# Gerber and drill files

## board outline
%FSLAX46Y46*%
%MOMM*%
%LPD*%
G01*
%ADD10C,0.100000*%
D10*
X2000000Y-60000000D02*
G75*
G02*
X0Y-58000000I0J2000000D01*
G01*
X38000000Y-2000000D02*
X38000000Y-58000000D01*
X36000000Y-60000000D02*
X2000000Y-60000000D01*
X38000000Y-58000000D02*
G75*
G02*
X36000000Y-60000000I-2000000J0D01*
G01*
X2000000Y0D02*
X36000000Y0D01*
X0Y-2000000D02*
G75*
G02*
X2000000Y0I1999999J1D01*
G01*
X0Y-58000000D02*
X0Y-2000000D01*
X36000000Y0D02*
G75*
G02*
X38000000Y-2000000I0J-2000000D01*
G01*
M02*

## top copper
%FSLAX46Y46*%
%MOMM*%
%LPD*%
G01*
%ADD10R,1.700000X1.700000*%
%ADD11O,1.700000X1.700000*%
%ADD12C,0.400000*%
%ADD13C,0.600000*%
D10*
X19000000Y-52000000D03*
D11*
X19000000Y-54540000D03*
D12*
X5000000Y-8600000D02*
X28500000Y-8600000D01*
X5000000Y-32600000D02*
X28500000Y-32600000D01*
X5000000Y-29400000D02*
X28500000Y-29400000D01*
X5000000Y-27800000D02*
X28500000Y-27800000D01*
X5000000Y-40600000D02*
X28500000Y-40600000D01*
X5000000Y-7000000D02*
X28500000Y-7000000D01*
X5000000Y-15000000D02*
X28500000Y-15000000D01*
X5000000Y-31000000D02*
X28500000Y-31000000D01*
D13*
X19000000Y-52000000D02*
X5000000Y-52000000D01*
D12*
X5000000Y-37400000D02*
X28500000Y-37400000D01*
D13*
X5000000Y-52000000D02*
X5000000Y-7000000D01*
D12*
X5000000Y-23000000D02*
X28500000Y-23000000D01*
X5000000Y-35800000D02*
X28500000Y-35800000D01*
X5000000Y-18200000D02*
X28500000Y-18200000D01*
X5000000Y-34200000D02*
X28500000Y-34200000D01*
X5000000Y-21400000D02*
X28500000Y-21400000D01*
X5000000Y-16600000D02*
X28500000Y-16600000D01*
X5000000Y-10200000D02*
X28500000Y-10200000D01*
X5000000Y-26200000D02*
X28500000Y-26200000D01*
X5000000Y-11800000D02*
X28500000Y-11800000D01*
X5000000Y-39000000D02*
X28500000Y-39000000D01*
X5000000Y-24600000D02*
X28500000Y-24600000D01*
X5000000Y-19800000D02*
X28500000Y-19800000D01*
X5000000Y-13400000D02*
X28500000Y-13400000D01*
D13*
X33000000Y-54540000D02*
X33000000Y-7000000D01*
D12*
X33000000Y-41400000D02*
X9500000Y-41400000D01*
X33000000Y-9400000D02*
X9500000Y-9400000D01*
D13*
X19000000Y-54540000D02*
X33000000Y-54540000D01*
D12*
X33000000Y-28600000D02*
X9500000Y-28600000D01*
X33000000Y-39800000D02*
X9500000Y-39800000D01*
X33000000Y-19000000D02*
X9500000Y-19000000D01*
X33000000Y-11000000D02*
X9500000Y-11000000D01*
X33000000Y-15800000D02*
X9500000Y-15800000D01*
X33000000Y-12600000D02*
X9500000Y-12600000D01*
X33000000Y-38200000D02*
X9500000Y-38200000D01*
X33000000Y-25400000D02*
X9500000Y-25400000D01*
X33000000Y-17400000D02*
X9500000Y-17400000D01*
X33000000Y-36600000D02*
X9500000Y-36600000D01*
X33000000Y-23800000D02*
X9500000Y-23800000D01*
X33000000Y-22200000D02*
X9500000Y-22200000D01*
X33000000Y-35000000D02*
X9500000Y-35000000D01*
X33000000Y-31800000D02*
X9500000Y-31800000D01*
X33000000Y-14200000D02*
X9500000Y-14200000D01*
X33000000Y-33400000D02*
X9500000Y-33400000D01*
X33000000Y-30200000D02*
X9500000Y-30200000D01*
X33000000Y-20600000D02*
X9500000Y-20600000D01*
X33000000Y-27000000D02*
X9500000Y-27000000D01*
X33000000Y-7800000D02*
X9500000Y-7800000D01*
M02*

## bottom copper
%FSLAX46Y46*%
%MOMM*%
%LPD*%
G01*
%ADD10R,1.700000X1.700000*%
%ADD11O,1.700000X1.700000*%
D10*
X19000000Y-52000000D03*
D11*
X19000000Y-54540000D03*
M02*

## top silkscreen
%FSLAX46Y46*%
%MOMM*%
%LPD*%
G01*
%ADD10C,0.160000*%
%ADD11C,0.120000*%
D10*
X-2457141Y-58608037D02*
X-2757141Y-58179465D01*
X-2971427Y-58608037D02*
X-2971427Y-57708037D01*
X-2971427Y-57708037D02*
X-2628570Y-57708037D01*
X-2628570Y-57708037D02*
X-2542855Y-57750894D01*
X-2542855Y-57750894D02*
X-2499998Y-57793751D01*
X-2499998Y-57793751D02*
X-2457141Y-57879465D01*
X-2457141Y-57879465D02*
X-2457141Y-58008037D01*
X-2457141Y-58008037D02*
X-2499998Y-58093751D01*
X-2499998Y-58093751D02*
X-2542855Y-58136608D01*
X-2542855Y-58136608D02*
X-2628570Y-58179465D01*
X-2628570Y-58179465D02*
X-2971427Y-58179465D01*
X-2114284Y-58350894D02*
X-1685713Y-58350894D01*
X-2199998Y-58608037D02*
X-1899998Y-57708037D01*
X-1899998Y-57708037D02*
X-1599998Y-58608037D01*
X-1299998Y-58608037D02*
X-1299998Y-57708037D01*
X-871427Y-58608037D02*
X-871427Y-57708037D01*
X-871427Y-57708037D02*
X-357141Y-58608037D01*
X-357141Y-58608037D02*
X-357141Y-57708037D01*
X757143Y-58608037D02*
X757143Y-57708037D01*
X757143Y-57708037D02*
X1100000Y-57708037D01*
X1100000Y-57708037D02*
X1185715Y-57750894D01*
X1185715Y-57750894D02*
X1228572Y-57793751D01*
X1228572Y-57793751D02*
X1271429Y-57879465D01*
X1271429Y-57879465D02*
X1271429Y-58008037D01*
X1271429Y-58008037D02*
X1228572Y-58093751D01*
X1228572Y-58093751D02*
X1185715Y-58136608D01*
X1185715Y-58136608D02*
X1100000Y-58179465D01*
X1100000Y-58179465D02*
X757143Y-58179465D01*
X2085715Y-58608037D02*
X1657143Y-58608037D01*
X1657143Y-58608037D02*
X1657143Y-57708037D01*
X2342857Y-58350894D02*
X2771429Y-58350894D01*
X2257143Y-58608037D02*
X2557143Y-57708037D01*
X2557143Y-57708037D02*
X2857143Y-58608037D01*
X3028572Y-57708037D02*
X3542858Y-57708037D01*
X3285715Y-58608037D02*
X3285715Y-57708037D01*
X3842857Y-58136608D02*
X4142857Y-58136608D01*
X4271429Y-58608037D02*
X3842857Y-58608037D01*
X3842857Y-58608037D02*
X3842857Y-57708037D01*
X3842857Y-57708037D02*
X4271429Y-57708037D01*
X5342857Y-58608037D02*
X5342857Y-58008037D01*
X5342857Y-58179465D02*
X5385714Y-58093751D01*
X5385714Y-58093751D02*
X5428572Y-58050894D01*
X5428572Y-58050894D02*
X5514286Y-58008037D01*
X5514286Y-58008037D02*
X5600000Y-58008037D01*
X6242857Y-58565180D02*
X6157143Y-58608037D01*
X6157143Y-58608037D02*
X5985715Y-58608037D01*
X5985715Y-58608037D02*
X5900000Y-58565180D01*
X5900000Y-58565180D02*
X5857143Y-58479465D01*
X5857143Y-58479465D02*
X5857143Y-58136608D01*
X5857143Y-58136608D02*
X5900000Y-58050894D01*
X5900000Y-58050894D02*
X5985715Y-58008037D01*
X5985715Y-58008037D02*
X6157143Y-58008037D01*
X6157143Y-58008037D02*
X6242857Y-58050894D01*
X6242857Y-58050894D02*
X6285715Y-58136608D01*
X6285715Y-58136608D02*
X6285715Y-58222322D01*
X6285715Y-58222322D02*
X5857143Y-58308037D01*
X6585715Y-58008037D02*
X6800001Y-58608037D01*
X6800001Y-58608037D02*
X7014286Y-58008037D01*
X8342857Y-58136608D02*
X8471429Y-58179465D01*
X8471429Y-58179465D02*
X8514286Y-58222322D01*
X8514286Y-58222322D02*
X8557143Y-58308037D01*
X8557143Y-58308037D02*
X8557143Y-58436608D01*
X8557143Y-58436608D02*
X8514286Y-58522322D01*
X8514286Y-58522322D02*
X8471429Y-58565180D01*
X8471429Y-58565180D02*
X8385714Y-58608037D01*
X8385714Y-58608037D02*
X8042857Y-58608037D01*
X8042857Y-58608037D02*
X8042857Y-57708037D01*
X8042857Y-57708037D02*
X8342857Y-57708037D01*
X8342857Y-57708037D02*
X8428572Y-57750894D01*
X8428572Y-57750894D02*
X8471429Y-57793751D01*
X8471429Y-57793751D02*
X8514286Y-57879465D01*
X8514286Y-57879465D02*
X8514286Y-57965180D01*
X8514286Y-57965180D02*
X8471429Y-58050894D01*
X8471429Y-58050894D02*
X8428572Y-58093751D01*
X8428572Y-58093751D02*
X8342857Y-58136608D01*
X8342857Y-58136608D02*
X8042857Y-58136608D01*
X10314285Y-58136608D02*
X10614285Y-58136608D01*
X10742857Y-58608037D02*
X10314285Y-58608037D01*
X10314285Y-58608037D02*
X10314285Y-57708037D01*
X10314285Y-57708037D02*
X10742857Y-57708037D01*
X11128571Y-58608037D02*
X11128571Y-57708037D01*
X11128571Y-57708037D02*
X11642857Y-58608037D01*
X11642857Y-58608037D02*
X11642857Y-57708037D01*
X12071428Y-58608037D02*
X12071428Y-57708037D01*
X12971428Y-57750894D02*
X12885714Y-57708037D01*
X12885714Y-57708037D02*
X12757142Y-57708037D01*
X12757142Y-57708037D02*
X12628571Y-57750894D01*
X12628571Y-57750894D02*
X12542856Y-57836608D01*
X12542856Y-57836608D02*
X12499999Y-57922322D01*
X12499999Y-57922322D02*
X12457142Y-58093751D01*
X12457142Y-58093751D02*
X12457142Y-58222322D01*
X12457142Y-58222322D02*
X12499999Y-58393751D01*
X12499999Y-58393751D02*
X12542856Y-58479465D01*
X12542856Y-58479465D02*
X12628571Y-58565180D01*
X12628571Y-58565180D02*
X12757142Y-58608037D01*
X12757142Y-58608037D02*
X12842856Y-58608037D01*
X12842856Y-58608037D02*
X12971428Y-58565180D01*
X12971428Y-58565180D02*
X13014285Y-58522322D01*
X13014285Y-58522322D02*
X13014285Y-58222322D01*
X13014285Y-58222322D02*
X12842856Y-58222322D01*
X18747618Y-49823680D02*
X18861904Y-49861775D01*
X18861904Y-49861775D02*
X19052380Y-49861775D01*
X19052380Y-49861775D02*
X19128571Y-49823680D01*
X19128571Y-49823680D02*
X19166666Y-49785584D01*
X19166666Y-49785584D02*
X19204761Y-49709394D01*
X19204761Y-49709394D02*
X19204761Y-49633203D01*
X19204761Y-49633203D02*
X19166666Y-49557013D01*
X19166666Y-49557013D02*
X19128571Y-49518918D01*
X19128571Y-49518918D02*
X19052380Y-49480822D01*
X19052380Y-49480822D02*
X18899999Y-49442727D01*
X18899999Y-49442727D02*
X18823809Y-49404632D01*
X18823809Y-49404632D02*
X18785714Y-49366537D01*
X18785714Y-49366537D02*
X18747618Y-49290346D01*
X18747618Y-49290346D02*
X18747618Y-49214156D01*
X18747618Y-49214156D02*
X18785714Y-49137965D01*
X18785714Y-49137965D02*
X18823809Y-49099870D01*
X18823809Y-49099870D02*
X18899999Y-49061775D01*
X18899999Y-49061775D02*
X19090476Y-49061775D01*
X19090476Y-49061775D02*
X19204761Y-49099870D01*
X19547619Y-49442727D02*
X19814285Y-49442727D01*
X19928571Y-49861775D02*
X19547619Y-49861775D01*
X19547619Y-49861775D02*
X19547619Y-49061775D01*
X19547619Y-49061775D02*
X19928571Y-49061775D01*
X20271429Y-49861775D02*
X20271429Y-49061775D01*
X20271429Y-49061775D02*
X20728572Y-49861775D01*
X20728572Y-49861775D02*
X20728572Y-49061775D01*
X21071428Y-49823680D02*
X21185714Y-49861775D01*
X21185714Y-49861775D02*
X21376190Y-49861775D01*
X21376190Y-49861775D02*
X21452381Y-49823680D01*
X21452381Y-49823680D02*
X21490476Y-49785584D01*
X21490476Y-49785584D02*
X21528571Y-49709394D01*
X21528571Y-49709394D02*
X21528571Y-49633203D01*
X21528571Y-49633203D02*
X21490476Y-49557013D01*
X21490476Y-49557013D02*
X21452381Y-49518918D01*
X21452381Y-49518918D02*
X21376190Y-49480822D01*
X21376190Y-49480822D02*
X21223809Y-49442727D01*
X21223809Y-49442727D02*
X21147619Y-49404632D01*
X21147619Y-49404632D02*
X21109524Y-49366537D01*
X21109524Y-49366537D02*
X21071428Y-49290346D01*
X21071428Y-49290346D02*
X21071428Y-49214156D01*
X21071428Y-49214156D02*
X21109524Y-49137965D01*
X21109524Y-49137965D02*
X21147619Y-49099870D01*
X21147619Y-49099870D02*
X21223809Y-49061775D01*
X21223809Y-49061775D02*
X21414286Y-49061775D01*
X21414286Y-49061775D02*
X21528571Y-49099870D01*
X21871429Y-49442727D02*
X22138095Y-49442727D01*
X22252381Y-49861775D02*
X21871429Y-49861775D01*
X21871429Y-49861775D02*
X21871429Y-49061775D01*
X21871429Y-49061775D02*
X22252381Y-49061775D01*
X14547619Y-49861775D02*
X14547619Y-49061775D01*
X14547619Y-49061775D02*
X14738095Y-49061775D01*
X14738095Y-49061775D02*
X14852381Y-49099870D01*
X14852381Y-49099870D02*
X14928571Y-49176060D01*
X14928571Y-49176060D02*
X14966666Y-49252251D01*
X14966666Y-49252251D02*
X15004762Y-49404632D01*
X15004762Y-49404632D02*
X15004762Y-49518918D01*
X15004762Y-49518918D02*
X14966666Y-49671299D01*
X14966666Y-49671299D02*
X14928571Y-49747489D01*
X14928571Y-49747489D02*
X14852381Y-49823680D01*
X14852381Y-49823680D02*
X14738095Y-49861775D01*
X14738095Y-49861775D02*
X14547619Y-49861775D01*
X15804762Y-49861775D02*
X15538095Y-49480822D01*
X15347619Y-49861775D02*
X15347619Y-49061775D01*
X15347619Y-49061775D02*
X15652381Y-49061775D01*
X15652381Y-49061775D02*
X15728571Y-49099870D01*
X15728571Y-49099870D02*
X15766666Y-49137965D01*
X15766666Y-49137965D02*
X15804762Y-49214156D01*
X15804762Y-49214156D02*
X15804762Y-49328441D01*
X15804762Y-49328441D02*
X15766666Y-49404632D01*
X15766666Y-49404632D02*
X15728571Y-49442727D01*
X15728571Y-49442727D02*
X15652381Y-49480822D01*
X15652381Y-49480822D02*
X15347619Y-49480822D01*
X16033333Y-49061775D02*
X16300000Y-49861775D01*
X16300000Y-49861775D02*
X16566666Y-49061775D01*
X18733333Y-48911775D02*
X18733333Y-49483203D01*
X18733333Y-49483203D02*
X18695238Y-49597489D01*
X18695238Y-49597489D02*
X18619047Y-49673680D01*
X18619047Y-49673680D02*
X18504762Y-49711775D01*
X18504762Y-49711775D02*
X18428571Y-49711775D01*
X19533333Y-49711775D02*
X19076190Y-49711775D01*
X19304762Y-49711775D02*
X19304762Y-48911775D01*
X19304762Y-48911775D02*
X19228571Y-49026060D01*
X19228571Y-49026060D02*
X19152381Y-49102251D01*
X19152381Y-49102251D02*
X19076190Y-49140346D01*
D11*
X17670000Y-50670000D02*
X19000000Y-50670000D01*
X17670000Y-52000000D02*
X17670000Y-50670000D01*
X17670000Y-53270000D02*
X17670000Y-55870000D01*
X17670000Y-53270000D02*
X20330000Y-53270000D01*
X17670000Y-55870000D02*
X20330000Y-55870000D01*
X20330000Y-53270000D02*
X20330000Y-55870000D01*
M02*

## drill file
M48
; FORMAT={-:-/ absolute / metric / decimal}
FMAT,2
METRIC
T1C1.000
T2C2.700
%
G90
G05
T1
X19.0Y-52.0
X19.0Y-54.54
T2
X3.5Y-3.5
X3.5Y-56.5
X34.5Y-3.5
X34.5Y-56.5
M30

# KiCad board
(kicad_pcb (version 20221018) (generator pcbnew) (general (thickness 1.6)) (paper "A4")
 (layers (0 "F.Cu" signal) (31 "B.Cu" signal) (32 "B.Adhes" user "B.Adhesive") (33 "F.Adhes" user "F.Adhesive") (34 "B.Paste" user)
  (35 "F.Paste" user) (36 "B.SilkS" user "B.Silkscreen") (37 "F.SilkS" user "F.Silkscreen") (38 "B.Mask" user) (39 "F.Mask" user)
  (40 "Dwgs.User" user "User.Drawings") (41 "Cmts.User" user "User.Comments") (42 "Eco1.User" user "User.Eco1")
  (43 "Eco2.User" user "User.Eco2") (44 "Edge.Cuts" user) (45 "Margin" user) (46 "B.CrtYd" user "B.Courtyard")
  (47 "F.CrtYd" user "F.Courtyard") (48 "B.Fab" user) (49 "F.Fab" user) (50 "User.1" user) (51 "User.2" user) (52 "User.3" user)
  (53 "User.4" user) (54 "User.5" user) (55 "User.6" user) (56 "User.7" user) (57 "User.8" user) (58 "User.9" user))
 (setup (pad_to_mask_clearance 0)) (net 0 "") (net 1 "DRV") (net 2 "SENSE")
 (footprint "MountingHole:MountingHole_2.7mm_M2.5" (layer "F.Cu") (at 3.5 56.5)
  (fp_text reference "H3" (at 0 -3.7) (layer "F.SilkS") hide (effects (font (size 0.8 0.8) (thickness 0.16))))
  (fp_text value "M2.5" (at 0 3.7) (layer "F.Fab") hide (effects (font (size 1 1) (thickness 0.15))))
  (pad "" np_thru_hole circle (at 0 0) (size 2.7 2.7) (drill 2.7) (layers "*.Cu" "*.Mask")))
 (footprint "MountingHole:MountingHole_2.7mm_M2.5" (layer "F.Cu") (at 3.5 3.5)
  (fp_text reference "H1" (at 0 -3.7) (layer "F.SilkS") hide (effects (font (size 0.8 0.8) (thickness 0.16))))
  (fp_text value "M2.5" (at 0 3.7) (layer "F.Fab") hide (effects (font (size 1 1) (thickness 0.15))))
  (pad "" np_thru_hole circle (at 0 0) (size 2.7 2.7) (drill 2.7) (layers "*.Cu" "*.Mask")))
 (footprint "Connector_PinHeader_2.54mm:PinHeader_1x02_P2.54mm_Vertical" (layer "F.Cu") (at 19 52)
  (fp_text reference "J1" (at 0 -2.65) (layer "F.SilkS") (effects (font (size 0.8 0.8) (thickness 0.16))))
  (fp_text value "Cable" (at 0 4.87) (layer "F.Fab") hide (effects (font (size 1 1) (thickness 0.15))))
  (fp_line (start -1.33 -1.33) (end 0 -1.33) (stroke (width 0.12) (type solid)) (layer "F.SilkS"))
  (fp_line (start -1.33 0) (end -1.33 -1.33) (stroke (width 0.12) (type solid)) (layer "F.SilkS"))
  (fp_line (start -1.33 1.27) (end -1.33 3.87) (stroke (width 0.12) (type solid)) (layer "F.SilkS"))
  (fp_line (start -1.33 1.27) (end 1.33 1.27) (stroke (width 0.12) (type solid)) (layer "F.SilkS"))
  (fp_line (start -1.33 3.87) (end 1.33 3.87) (stroke (width 0.12) (type solid)) (layer "F.SilkS"))
  (fp_line (start 1.33 1.27) (end 1.33 3.87) (stroke (width 0.12) (type solid)) (layer "F.SilkS"))
  (pad "1" thru_hole rect (at 0 0) (size 1.7 1.7) (drill 1) (layers "*.Cu" "*.Mask") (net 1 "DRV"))
  (pad "2" thru_hole oval (at 0 2.54) (size 1.7 1.7) (drill 1) (layers "*.Cu" "*.Mask") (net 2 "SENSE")))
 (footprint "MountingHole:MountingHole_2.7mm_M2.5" (layer "F.Cu") (at 34.5 3.5)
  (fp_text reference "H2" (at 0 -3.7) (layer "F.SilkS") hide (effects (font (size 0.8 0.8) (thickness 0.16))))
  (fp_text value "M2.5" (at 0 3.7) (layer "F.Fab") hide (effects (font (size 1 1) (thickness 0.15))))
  (pad "" np_thru_hole circle (at 0 0) (size 2.7 2.7) (drill 2.7) (layers "*.Cu" "*.Mask")))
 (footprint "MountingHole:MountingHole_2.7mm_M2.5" (layer "F.Cu") (at 34.5 56.5)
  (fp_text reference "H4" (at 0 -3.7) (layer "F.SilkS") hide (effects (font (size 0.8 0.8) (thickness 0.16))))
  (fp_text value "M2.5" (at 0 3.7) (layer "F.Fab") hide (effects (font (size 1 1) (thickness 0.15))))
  (pad "" np_thru_hole circle (at 0 0) (size 2.7 2.7) (drill 2.7) (layers "*.Cu" "*.Mask")))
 (gr_arc (start 2 60) (mid 0.585786 59.414213) (end 0 58) (stroke (width 0.1) (type default)) (layer "Edge.Cuts"))
 (gr_line (start 38 2) (end 38 58) (stroke (width 0.1) (type default)) (layer "Edge.Cuts"))
 (gr_line (start 36 60) (end 2 60) (stroke (width 0.1) (type default)) (layer "Edge.Cuts"))
 (gr_arc (start 38 58) (mid 37.414213 59.414213) (end 36 60) (stroke (width 0.1) (type default)) (layer "Edge.Cuts"))
 (gr_line (start 2 0) (end 36 0) (stroke (width 0.1) (type default)) (layer "Edge.Cuts"))
 (gr_arc (start 0 2) (mid 0.585786 0.585786) (end 2 0) (stroke (width 0.1) (type default)) (layer "Edge.Cuts"))
 (gr_line (start 0 58) (end 0 2) (stroke (width 0.1) (type default)) (layer "Edge.Cuts"))
 (gr_arc (start 36 0) (mid 37.414213 0.585786) (end 38 2) (stroke (width 0.1) (type default)) (layer "Edge.Cuts"))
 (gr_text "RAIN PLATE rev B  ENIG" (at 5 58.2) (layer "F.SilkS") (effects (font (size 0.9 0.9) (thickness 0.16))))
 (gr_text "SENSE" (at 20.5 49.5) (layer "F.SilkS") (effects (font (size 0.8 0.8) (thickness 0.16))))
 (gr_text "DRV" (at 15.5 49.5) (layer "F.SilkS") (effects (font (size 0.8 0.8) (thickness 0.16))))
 (segment (start 5 8.6) (end 28.5 8.6) (width 0.4) (layer "F.Cu") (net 1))
 (segment (start 5 32.6) (end 28.5 32.6) (width 0.4) (layer "F.Cu") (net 1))
 (segment (start 5 29.4) (end 28.5 29.4) (width 0.4) (layer "F.Cu") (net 1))
 (segment (start 5 27.8) (end 28.5 27.8) (width 0.4) (layer "F.Cu") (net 1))
 (segment (start 5 40.6) (end 28.5 40.6) (width 0.4) (layer "F.Cu") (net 1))
 (segment (start 5 7) (end 28.5 7) (width 0.4) (layer "F.Cu") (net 1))
 (segment (start 5 15) (end 28.5 15) (width 0.4) (layer "F.Cu") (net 1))
 (segment (start 5 31) (end 28.5 31) (width 0.4) (layer "F.Cu") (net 1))
 (segment (start 19 52) (end 5 52) (width 0.6) (layer "F.Cu") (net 1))
 (segment (start 5 37.4) (end 28.5 37.4) (width 0.4) (layer "F.Cu") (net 1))
 (segment (start 5 52) (end 5 7) (width 0.6) (layer "F.Cu") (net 1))
 (segment (start 5 23) (end 28.5 23) (width 0.4) (layer "F.Cu") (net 1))
 (segment (start 5 35.8) (end 28.5 35.8) (width 0.4) (layer "F.Cu") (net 1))
 (segment (start 5 18.2) (end 28.5 18.2) (width 0.4) (layer "F.Cu") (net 1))
 (segment (start 5 34.2) (end 28.5 34.2) (width 0.4) (layer "F.Cu") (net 1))
 (segment (start 5 21.4) (end 28.5 21.4) (width 0.4) (layer "F.Cu") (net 1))
 (segment (start 5 16.6) (end 28.5 16.6) (width 0.4) (layer "F.Cu") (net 1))
 (segment (start 5 10.2) (end 28.5 10.2) (width 0.4) (layer "F.Cu") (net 1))
 (segment (start 5 26.2) (end 28.5 26.2) (width 0.4) (layer "F.Cu") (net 1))
 (segment (start 5 11.8) (end 28.5 11.8) (width 0.4) (layer "F.Cu") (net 1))
 (segment (start 5 39) (end 28.5 39) (width 0.4) (layer "F.Cu") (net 1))
 (segment (start 5 24.6) (end 28.5 24.6) (width 0.4) (layer "F.Cu") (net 1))
 (segment (start 5 19.8) (end 28.5 19.8) (width 0.4) (layer "F.Cu") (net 1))
 (segment (start 5 13.4) (end 28.5 13.4) (width 0.4) (layer "F.Cu") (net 1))
 (segment (start 33 54.54) (end 33 7) (width 0.6) (layer "F.Cu") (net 2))
 (segment (start 33 41.4) (end 9.5 41.4) (width 0.4) (layer "F.Cu") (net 2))
 (segment (start 33 9.4) (end 9.5 9.4) (width 0.4) (layer "F.Cu") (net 2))
 (segment (start 19 54.54) (end 33 54.54) (width 0.6) (layer "F.Cu") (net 2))
 (segment (start 33 28.6) (end 9.5 28.6) (width 0.4) (layer "F.Cu") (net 2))
 (segment (start 33 39.8) (end 9.5 39.8) (width 0.4) (layer "F.Cu") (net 2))
 (segment (start 33 19) (end 9.5 19) (width 0.4) (layer "F.Cu") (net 2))
 (segment (start 33 11) (end 9.5 11) (width 0.4) (layer "F.Cu") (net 2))
 (segment (start 33 15.8) (end 9.5 15.8) (width 0.4) (layer "F.Cu") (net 2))
 (segment (start 33 12.6) (end 9.5 12.6) (width 0.4) (layer "F.Cu") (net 2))
 (segment (start 33 38.2) (end 9.5 38.2) (width 0.4) (layer "F.Cu") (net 2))
 (segment (start 33 25.4) (end 9.5 25.4) (width 0.4) (layer "F.Cu") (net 2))
 (segment (start 33 17.4) (end 9.5 17.4) (width 0.4) (layer "F.Cu") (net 2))
 (segment (start 33 36.6) (end 9.5 36.6) (width 0.4) (layer "F.Cu") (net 2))
 (segment (start 33 23.8) (end 9.5 23.8) (width 0.4) (layer "F.Cu") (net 2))
 (segment (start 33 22.2) (end 9.5 22.2) (width 0.4) (layer "F.Cu") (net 2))
 (segment (start 33 35) (end 9.5 35) (width 0.4) (layer "F.Cu") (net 2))
 (segment (start 33 31.8) (end 9.5 31.8) (width 0.4) (layer "F.Cu") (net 2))
 (segment (start 33 14.2) (end 9.5 14.2) (width 0.4) (layer "F.Cu") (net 2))
 (segment (start 33 33.4) (end 9.5 33.4) (width 0.4) (layer "F.Cu") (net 2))
 (segment (start 33 30.2) (end 9.5 30.2) (width 0.4) (layer "F.Cu") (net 2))
 (segment (start 33 20.6) (end 9.5 20.6) (width 0.4) (layer "F.Cu") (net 2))
 (segment (start 33 27) (end 9.5 27) (width 0.4) (layer "F.Cu") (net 2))
 (segment (start 33 7.8) (end 9.5 7.8) (width 0.4) (layer "F.Cu") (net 2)))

